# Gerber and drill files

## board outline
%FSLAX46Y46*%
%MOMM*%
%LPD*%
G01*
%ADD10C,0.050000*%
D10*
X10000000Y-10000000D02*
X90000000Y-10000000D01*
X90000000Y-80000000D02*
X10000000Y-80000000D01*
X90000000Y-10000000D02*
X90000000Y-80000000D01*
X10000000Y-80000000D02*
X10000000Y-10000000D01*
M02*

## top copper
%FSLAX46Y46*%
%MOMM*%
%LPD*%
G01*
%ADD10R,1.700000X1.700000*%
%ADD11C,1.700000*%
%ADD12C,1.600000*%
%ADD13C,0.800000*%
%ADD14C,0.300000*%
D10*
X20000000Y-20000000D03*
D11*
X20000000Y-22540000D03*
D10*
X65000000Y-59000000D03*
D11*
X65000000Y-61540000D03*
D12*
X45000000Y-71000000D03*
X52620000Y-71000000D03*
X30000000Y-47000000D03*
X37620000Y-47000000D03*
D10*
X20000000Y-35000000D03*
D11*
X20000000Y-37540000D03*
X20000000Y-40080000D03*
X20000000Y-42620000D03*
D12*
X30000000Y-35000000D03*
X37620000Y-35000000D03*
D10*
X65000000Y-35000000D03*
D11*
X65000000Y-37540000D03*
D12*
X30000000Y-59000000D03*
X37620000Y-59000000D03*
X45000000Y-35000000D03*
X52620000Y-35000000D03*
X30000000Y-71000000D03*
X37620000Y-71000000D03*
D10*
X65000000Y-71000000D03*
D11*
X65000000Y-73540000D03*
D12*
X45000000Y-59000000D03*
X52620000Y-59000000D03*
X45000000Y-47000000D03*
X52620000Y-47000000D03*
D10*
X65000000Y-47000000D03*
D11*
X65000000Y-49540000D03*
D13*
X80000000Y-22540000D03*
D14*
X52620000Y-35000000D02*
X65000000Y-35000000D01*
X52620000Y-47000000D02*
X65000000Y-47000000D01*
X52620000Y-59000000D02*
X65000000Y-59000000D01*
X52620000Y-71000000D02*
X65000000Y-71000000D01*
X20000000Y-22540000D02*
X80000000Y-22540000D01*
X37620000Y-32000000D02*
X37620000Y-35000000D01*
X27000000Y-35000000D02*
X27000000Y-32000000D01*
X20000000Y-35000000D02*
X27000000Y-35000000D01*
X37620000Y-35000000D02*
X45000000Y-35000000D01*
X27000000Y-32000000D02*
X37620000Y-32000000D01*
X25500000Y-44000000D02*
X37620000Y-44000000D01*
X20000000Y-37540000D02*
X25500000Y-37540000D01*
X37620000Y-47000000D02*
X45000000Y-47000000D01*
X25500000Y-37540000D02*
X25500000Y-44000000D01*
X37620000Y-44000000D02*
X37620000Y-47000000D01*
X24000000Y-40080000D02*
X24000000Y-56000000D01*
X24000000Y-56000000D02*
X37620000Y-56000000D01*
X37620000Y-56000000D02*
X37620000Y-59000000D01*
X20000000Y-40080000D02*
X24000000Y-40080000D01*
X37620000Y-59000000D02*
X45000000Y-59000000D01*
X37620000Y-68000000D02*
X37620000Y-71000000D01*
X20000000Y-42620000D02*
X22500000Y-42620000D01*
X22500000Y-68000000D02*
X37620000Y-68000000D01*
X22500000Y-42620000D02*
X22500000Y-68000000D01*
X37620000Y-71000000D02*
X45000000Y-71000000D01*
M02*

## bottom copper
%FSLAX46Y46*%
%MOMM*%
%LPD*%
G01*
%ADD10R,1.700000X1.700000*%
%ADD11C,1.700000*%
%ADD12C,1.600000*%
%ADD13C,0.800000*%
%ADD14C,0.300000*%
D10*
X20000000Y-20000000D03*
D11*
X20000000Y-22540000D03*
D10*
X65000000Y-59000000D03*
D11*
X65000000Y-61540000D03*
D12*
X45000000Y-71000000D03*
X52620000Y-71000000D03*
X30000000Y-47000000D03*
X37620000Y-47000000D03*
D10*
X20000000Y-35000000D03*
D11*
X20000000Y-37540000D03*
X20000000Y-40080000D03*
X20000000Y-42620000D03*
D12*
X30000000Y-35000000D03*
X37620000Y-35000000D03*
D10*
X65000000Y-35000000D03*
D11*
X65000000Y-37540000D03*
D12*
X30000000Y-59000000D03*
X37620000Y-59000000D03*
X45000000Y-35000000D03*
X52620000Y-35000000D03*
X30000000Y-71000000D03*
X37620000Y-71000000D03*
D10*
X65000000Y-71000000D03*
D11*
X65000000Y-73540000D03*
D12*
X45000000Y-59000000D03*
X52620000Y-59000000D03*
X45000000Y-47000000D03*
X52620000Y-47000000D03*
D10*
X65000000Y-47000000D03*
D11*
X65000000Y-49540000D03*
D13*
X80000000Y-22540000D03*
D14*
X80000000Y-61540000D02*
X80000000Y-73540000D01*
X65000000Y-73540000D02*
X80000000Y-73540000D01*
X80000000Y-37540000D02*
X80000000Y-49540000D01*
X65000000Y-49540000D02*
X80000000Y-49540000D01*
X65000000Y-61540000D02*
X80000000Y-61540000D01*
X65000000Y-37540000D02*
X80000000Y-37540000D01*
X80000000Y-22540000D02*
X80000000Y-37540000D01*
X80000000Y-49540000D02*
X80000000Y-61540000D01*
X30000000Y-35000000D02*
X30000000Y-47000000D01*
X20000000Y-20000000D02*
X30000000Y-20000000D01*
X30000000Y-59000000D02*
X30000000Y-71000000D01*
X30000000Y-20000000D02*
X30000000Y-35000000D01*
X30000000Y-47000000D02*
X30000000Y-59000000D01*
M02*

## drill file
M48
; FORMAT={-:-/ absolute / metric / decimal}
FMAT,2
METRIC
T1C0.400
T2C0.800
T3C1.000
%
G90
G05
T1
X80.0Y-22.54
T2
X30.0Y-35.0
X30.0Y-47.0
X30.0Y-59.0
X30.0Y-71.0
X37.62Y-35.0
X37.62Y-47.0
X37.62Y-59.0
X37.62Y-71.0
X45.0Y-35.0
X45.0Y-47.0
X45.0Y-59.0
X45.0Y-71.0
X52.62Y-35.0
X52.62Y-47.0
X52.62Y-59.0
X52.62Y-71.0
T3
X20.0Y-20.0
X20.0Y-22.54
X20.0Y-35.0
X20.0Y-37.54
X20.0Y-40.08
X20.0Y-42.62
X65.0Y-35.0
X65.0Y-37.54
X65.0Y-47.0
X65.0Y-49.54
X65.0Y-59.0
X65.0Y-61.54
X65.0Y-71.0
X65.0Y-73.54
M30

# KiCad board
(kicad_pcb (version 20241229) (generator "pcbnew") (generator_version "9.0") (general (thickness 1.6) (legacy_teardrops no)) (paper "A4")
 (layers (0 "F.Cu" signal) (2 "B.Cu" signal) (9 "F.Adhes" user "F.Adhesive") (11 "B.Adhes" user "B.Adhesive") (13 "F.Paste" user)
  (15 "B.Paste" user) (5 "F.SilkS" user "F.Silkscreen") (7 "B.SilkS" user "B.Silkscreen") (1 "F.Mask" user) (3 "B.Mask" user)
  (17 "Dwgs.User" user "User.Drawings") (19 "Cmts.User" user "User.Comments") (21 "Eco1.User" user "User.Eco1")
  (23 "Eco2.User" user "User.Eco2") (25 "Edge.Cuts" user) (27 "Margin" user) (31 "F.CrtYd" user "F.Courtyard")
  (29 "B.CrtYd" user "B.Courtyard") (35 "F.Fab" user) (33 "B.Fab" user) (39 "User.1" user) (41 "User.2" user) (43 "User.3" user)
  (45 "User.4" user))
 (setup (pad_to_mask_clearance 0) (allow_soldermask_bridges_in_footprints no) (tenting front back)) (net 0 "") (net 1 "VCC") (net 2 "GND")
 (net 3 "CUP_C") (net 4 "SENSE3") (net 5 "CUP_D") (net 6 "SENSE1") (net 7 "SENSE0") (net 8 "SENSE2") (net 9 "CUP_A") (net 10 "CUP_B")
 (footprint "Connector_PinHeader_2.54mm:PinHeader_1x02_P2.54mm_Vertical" (layer "F.Cu") (at 20 20)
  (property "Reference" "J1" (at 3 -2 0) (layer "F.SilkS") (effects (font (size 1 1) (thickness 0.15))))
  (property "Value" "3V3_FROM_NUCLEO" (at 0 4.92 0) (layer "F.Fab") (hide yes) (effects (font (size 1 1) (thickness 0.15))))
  (pad "1" thru_hole rect (at 0 0) (size 1.7 1.7) (drill 1) (layers "*.Cu" "*.Mask") (remove_unused_layers no) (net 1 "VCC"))
  (pad "2" thru_hole circle (at 0 2.54) (size 1.7 1.7) (drill 1) (layers "*.Cu" "*.Mask") (remove_unused_layers no) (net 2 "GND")))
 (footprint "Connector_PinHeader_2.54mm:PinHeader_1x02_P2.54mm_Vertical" (layer "F.Cu") (at 65 59)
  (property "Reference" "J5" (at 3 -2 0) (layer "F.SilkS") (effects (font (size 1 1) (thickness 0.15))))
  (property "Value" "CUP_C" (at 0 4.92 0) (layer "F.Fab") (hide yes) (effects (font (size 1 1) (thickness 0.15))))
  (pad "1" thru_hole rect (at 0 0) (size 1.7 1.7) (drill 1) (layers "*.Cu" "*.Mask") (remove_unused_layers no) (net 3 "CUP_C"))
  (pad "2" thru_hole circle (at 0 2.54) (size 1.7 1.7) (drill 1) (layers "*.Cu" "*.Mask") (remove_unused_layers no) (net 2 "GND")))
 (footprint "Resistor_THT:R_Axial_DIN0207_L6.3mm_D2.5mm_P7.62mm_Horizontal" (layer "F.Cu") (at 45 71)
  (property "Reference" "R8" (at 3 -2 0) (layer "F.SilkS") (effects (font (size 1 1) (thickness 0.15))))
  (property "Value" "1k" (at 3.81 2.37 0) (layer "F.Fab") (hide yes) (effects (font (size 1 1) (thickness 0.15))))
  (pad "1" thru_hole circle (at 0 0) (size 1.6 1.6) (drill 0.8) (layers "*.Cu" "*.Mask") (remove_unused_layers no) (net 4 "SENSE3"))
  (pad "2" thru_hole circle (at 7.62 0) (size 1.6 1.6) (drill 0.8) (layers "*.Cu" "*.Mask") (remove_unused_layers no) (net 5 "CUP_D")))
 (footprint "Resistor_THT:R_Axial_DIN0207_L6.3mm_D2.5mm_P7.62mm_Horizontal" (layer "F.Cu") (at 30 47)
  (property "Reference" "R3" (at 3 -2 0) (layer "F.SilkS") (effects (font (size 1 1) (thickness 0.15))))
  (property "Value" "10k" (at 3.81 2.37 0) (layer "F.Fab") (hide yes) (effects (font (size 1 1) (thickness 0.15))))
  (pad "1" thru_hole circle (at 0 0) (size 1.6 1.6) (drill 0.8) (layers "*.Cu" "*.Mask") (remove_unused_layers no) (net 1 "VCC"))
  (pad "2" thru_hole circle (at 7.62 0) (size 1.6 1.6) (drill 0.8) (layers "*.Cu" "*.Mask") (remove_unused_layers no) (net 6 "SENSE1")))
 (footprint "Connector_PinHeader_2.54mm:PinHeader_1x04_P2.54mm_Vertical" (layer "F.Cu") (at 20 35)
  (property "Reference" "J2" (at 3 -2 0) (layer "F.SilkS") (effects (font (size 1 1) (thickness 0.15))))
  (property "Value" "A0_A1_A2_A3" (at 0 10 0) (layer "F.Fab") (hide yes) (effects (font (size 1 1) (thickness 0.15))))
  (pad "1" thru_hole rect (at 0 0) (size 1.7 1.7) (drill 1) (layers "*.Cu" "*.Mask") (remove_unused_layers no) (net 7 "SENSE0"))
  (pad "2" thru_hole circle (at 0 2.54) (size 1.7 1.7) (drill 1) (layers "*.Cu" "*.Mask") (remove_unused_layers no) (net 6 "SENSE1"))
  (pad "3" thru_hole circle (at 0 5.08) (size 1.7 1.7) (drill 1) (layers "*.Cu" "*.Mask") (remove_unused_layers no) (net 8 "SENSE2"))
  (pad "4" thru_hole circle (at 0 7.62) (size 1.7 1.7) (drill 1) (layers "*.Cu" "*.Mask") (remove_unused_layers no) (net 4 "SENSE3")))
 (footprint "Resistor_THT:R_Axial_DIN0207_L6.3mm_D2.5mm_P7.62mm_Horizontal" (layer "F.Cu") (at 30 35)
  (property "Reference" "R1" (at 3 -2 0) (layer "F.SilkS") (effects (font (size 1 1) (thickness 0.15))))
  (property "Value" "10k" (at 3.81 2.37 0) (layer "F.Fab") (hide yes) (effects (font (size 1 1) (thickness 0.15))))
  (pad "1" thru_hole circle (at 0 0) (size 1.6 1.6) (drill 0.8) (layers "*.Cu" "*.Mask") (remove_unused_layers no) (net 1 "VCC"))
  (pad "2" thru_hole circle (at 7.62 0) (size 1.6 1.6) (drill 0.8) (layers "*.Cu" "*.Mask") (remove_unused_layers no) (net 7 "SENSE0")))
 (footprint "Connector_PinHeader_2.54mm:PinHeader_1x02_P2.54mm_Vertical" (layer "F.Cu") (at 65 35)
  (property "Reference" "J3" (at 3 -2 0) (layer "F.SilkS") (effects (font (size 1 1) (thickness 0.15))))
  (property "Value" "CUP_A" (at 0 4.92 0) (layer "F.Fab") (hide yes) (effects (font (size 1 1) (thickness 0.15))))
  (pad "1" thru_hole rect (at 0 0) (size 1.7 1.7) (drill 1) (layers "*.Cu" "*.Mask") (remove_unused_layers no) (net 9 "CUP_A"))
  (pad "2" thru_hole circle (at 0 2.54) (size 1.7 1.7) (drill 1) (layers "*.Cu" "*.Mask") (remove_unused_layers no) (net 2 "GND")))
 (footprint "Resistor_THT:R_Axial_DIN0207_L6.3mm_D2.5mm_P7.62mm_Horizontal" (layer "F.Cu") (at 30 59)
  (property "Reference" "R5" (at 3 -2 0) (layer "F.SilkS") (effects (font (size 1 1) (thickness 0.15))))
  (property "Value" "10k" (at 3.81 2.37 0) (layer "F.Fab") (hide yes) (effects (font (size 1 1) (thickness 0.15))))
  (pad "1" thru_hole circle (at 0 0) (size 1.6 1.6) (drill 0.8) (layers "*.Cu" "*.Mask") (remove_unused_layers no) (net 1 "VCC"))
  (pad "2" thru_hole circle (at 7.62 0) (size 1.6 1.6) (drill 0.8) (layers "*.Cu" "*.Mask") (remove_unused_layers no) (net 8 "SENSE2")))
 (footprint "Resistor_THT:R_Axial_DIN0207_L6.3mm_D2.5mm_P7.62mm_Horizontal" (layer "F.Cu") (at 45 35)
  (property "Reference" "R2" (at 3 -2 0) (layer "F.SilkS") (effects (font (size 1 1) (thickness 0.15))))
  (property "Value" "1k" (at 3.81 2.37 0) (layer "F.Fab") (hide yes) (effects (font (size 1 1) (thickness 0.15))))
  (pad "1" thru_hole circle (at 0 0) (size 1.6 1.6) (drill 0.8) (layers "*.Cu" "*.Mask") (remove_unused_layers no) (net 7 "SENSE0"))
  (pad "2" thru_hole circle (at 7.62 0) (size 1.6 1.6) (drill 0.8) (layers "*.Cu" "*.Mask") (remove_unused_layers no) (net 9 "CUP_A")))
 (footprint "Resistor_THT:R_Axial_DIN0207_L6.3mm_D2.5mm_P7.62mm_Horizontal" (layer "F.Cu") (at 30 71)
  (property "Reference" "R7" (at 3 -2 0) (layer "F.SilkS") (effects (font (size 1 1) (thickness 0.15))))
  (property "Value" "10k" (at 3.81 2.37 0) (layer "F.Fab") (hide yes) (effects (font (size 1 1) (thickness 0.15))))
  (pad "1" thru_hole circle (at 0 0) (size 1.6 1.6) (drill 0.8) (layers "*.Cu" "*.Mask") (remove_unused_layers no) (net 1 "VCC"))
  (pad "2" thru_hole circle (at 7.62 0) (size 1.6 1.6) (drill 0.8) (layers "*.Cu" "*.Mask") (remove_unused_layers no) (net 4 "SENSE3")))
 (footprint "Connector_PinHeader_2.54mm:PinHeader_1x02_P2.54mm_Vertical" (layer "F.Cu") (at 65 71)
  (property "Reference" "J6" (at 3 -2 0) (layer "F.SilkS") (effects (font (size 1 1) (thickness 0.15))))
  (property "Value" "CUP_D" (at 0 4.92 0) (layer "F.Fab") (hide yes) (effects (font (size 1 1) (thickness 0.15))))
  (pad "1" thru_hole rect (at 0 0) (size 1.7 1.7) (drill 1) (layers "*.Cu" "*.Mask") (remove_unused_layers no) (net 5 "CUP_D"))
  (pad "2" thru_hole circle (at 0 2.54) (size 1.7 1.7) (drill 1) (layers "*.Cu" "*.Mask") (remove_unused_layers no) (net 2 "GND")))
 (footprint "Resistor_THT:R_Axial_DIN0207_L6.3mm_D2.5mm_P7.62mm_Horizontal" (layer "F.Cu") (at 45 59)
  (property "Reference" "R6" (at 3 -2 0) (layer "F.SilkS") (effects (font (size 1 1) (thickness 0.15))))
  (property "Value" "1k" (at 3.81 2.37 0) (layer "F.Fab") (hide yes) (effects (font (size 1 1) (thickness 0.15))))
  (pad "1" thru_hole circle (at 0 0) (size 1.6 1.6) (drill 0.8) (layers "*.Cu" "*.Mask") (remove_unused_layers no) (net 8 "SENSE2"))
  (pad "2" thru_hole circle (at 7.62 0) (size 1.6 1.6) (drill 0.8) (layers "*.Cu" "*.Mask") (remove_unused_layers no) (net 3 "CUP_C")))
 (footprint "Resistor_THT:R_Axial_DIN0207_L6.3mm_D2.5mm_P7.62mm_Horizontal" (layer "F.Cu") (at 45 47)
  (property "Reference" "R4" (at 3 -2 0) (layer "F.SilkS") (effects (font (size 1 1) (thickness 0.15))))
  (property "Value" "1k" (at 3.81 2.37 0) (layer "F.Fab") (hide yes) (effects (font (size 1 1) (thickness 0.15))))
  (pad "1" thru_hole circle (at 0 0) (size 1.6 1.6) (drill 0.8) (layers "*.Cu" "*.Mask") (remove_unused_layers no) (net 6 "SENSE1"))
  (pad "2" thru_hole circle (at 7.62 0) (size 1.6 1.6) (drill 0.8) (layers "*.Cu" "*.Mask") (remove_unused_layers no) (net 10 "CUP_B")))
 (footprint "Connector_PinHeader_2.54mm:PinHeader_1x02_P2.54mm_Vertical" (layer "F.Cu") (at 65 47)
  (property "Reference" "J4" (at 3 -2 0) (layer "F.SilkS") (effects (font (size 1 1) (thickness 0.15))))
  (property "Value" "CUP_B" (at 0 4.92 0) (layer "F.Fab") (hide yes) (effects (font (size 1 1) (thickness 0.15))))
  (pad "1" thru_hole rect (at 0 0) (size 1.7 1.7) (drill 1) (layers "*.Cu" "*.Mask") (remove_unused_layers no) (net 10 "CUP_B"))
  (pad "2" thru_hole circle (at 0 2.54) (size 1.7 1.7) (drill 1) (layers "*.Cu" "*.Mask") (remove_unused_layers no) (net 2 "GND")))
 (gr_line (start 10 10) (end 90 10) (stroke (width 0.05) (type default)) (layer "Edge.Cuts"))
 (gr_line (start 90 80) (end 10 80) (stroke (width 0.05) (type default)) (layer "Edge.Cuts"))
 (gr_line (start 90 10) (end 90 80) (stroke (width 0.05) (type default)) (layer "Edge.Cuts"))
 (gr_line (start 10 80) (end 10 10) (stroke (width 0.05) (type default)) (layer "Edge.Cuts"))
 (segment (start 52.62 35) (end 65 35) (width 0.3) (layer "F.Cu") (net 9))
 (segment (start 52.62 47) (end 65 47) (width 0.3) (layer "F.Cu") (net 10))
 (segment (start 52.62 59) (end 65 59) (width 0.3) (layer "F.Cu") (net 3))
 (segment (start 52.62 71) (end 65 71) (width 0.3) (layer "F.Cu") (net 5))
 (segment (start 20 22.54) (end 80 22.54) (width 0.3) (layer "F.Cu") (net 2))
 (via (at 80 22.54) (size 0.8) (drill 0.4) (layers "F.Cu" "B.Cu") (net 2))
 (segment (start 80 61.54) (end 80 73.54) (width 0.3) (layer "B.Cu") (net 2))
 (segment (start 65 73.54) (end 80 73.54) (width 0.3) (layer "B.Cu") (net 2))
 (segment (start 80 37.54) (end 80 49.54) (width 0.3) (layer "B.Cu") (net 2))
 (segment (start 65 49.54) (end 80 49.54) (width 0.3) (layer "B.Cu") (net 2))
 (segment (start 65 61.54) (end 80 61.54) (width 0.3) (layer "B.Cu") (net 2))
 (segment (start 65 37.54) (end 80 37.54) (width 0.3) (layer "B.Cu") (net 2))
 (segment (start 80 22.54) (end 80 37.54) (width 0.3) (layer "B.Cu") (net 2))
 (segment (start 80 49.54) (end 80 61.54) (width 0.3) (layer "B.Cu") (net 2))
 (segment (start 37.62 32) (end 37.62 35) (width 0.3) (layer "F.Cu") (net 7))
 (segment (start 27 35) (end 27 32) (width 0.3) (layer "F.Cu") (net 7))
 (segment (start 20 35) (end 27 35) (width 0.3) (layer "F.Cu") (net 7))
 (segment (start 37.62 35) (end 45 35) (width 0.3) (layer "F.Cu") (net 7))
 (segment (start 27 32) (end 37.62 32) (width 0.3) (layer "F.Cu") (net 7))
 (segment (start 25.5 44) (end 37.62 44) (width 0.3) (layer "F.Cu") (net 6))
 (segment (start 20 37.54) (end 25.5 37.54) (width 0.3) (layer "F.Cu") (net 6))
 (segment (start 37.62 47) (end 45 47) (width 0.3) (layer "F.Cu") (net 6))
 (segment (start 25.5 37.54) (end 25.5 44) (width 0.3) (layer "F.Cu") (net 6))
 (segment (start 37.62 44) (end 37.62 47) (width 0.3) (layer "F.Cu") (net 6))
 (segment (start 24 40.08) (end 24 56) (width 0.3) (layer "F.Cu") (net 8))
 (segment (start 24 56) (end 37.62 56) (width 0.3) (layer "F.Cu") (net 8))
 (segment (start 37.62 56) (end 37.62 59) (width 0.3) (layer "F.Cu") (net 8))
 (segment (start 20 40.08) (end 24 40.08) (width 0.3) (layer "F.Cu") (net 8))
 (segment (start 37.62 59) (end 45 59) (width 0.3) (layer "F.Cu") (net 8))
 (segment (start 37.62 68) (end 37.62 71) (width 0.3) (layer "F.Cu") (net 4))
 (segment (start 20 42.62) (end 22.5 42.62) (width 0.3) (layer "F.Cu") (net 4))
 (segment (start 22.5 68) (end 37.62 68) (width 0.3) (layer "F.Cu") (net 4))
 (segment (start 22.5 42.62) (end 22.5 68) (width 0.3) (layer "F.Cu") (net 4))
 (segment (start 37.62 71) (end 45 71) (width 0.3) (layer "F.Cu") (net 4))
 (segment (start 30 35) (end 30 47) (width 0.3) (layer "B.Cu") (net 1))
 (segment (start 20 20) (end 30 20) (width 0.3) (layer "B.Cu") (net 1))
 (segment (start 30 59) (end 30 71) (width 0.3) (layer "B.Cu") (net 1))
 (segment (start 30 20) (end 30 35) (width 0.3) (layer "B.Cu") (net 1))
 (segment (start 30 47) (end 30 59) (width 0.3) (layer "B.Cu") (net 1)))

